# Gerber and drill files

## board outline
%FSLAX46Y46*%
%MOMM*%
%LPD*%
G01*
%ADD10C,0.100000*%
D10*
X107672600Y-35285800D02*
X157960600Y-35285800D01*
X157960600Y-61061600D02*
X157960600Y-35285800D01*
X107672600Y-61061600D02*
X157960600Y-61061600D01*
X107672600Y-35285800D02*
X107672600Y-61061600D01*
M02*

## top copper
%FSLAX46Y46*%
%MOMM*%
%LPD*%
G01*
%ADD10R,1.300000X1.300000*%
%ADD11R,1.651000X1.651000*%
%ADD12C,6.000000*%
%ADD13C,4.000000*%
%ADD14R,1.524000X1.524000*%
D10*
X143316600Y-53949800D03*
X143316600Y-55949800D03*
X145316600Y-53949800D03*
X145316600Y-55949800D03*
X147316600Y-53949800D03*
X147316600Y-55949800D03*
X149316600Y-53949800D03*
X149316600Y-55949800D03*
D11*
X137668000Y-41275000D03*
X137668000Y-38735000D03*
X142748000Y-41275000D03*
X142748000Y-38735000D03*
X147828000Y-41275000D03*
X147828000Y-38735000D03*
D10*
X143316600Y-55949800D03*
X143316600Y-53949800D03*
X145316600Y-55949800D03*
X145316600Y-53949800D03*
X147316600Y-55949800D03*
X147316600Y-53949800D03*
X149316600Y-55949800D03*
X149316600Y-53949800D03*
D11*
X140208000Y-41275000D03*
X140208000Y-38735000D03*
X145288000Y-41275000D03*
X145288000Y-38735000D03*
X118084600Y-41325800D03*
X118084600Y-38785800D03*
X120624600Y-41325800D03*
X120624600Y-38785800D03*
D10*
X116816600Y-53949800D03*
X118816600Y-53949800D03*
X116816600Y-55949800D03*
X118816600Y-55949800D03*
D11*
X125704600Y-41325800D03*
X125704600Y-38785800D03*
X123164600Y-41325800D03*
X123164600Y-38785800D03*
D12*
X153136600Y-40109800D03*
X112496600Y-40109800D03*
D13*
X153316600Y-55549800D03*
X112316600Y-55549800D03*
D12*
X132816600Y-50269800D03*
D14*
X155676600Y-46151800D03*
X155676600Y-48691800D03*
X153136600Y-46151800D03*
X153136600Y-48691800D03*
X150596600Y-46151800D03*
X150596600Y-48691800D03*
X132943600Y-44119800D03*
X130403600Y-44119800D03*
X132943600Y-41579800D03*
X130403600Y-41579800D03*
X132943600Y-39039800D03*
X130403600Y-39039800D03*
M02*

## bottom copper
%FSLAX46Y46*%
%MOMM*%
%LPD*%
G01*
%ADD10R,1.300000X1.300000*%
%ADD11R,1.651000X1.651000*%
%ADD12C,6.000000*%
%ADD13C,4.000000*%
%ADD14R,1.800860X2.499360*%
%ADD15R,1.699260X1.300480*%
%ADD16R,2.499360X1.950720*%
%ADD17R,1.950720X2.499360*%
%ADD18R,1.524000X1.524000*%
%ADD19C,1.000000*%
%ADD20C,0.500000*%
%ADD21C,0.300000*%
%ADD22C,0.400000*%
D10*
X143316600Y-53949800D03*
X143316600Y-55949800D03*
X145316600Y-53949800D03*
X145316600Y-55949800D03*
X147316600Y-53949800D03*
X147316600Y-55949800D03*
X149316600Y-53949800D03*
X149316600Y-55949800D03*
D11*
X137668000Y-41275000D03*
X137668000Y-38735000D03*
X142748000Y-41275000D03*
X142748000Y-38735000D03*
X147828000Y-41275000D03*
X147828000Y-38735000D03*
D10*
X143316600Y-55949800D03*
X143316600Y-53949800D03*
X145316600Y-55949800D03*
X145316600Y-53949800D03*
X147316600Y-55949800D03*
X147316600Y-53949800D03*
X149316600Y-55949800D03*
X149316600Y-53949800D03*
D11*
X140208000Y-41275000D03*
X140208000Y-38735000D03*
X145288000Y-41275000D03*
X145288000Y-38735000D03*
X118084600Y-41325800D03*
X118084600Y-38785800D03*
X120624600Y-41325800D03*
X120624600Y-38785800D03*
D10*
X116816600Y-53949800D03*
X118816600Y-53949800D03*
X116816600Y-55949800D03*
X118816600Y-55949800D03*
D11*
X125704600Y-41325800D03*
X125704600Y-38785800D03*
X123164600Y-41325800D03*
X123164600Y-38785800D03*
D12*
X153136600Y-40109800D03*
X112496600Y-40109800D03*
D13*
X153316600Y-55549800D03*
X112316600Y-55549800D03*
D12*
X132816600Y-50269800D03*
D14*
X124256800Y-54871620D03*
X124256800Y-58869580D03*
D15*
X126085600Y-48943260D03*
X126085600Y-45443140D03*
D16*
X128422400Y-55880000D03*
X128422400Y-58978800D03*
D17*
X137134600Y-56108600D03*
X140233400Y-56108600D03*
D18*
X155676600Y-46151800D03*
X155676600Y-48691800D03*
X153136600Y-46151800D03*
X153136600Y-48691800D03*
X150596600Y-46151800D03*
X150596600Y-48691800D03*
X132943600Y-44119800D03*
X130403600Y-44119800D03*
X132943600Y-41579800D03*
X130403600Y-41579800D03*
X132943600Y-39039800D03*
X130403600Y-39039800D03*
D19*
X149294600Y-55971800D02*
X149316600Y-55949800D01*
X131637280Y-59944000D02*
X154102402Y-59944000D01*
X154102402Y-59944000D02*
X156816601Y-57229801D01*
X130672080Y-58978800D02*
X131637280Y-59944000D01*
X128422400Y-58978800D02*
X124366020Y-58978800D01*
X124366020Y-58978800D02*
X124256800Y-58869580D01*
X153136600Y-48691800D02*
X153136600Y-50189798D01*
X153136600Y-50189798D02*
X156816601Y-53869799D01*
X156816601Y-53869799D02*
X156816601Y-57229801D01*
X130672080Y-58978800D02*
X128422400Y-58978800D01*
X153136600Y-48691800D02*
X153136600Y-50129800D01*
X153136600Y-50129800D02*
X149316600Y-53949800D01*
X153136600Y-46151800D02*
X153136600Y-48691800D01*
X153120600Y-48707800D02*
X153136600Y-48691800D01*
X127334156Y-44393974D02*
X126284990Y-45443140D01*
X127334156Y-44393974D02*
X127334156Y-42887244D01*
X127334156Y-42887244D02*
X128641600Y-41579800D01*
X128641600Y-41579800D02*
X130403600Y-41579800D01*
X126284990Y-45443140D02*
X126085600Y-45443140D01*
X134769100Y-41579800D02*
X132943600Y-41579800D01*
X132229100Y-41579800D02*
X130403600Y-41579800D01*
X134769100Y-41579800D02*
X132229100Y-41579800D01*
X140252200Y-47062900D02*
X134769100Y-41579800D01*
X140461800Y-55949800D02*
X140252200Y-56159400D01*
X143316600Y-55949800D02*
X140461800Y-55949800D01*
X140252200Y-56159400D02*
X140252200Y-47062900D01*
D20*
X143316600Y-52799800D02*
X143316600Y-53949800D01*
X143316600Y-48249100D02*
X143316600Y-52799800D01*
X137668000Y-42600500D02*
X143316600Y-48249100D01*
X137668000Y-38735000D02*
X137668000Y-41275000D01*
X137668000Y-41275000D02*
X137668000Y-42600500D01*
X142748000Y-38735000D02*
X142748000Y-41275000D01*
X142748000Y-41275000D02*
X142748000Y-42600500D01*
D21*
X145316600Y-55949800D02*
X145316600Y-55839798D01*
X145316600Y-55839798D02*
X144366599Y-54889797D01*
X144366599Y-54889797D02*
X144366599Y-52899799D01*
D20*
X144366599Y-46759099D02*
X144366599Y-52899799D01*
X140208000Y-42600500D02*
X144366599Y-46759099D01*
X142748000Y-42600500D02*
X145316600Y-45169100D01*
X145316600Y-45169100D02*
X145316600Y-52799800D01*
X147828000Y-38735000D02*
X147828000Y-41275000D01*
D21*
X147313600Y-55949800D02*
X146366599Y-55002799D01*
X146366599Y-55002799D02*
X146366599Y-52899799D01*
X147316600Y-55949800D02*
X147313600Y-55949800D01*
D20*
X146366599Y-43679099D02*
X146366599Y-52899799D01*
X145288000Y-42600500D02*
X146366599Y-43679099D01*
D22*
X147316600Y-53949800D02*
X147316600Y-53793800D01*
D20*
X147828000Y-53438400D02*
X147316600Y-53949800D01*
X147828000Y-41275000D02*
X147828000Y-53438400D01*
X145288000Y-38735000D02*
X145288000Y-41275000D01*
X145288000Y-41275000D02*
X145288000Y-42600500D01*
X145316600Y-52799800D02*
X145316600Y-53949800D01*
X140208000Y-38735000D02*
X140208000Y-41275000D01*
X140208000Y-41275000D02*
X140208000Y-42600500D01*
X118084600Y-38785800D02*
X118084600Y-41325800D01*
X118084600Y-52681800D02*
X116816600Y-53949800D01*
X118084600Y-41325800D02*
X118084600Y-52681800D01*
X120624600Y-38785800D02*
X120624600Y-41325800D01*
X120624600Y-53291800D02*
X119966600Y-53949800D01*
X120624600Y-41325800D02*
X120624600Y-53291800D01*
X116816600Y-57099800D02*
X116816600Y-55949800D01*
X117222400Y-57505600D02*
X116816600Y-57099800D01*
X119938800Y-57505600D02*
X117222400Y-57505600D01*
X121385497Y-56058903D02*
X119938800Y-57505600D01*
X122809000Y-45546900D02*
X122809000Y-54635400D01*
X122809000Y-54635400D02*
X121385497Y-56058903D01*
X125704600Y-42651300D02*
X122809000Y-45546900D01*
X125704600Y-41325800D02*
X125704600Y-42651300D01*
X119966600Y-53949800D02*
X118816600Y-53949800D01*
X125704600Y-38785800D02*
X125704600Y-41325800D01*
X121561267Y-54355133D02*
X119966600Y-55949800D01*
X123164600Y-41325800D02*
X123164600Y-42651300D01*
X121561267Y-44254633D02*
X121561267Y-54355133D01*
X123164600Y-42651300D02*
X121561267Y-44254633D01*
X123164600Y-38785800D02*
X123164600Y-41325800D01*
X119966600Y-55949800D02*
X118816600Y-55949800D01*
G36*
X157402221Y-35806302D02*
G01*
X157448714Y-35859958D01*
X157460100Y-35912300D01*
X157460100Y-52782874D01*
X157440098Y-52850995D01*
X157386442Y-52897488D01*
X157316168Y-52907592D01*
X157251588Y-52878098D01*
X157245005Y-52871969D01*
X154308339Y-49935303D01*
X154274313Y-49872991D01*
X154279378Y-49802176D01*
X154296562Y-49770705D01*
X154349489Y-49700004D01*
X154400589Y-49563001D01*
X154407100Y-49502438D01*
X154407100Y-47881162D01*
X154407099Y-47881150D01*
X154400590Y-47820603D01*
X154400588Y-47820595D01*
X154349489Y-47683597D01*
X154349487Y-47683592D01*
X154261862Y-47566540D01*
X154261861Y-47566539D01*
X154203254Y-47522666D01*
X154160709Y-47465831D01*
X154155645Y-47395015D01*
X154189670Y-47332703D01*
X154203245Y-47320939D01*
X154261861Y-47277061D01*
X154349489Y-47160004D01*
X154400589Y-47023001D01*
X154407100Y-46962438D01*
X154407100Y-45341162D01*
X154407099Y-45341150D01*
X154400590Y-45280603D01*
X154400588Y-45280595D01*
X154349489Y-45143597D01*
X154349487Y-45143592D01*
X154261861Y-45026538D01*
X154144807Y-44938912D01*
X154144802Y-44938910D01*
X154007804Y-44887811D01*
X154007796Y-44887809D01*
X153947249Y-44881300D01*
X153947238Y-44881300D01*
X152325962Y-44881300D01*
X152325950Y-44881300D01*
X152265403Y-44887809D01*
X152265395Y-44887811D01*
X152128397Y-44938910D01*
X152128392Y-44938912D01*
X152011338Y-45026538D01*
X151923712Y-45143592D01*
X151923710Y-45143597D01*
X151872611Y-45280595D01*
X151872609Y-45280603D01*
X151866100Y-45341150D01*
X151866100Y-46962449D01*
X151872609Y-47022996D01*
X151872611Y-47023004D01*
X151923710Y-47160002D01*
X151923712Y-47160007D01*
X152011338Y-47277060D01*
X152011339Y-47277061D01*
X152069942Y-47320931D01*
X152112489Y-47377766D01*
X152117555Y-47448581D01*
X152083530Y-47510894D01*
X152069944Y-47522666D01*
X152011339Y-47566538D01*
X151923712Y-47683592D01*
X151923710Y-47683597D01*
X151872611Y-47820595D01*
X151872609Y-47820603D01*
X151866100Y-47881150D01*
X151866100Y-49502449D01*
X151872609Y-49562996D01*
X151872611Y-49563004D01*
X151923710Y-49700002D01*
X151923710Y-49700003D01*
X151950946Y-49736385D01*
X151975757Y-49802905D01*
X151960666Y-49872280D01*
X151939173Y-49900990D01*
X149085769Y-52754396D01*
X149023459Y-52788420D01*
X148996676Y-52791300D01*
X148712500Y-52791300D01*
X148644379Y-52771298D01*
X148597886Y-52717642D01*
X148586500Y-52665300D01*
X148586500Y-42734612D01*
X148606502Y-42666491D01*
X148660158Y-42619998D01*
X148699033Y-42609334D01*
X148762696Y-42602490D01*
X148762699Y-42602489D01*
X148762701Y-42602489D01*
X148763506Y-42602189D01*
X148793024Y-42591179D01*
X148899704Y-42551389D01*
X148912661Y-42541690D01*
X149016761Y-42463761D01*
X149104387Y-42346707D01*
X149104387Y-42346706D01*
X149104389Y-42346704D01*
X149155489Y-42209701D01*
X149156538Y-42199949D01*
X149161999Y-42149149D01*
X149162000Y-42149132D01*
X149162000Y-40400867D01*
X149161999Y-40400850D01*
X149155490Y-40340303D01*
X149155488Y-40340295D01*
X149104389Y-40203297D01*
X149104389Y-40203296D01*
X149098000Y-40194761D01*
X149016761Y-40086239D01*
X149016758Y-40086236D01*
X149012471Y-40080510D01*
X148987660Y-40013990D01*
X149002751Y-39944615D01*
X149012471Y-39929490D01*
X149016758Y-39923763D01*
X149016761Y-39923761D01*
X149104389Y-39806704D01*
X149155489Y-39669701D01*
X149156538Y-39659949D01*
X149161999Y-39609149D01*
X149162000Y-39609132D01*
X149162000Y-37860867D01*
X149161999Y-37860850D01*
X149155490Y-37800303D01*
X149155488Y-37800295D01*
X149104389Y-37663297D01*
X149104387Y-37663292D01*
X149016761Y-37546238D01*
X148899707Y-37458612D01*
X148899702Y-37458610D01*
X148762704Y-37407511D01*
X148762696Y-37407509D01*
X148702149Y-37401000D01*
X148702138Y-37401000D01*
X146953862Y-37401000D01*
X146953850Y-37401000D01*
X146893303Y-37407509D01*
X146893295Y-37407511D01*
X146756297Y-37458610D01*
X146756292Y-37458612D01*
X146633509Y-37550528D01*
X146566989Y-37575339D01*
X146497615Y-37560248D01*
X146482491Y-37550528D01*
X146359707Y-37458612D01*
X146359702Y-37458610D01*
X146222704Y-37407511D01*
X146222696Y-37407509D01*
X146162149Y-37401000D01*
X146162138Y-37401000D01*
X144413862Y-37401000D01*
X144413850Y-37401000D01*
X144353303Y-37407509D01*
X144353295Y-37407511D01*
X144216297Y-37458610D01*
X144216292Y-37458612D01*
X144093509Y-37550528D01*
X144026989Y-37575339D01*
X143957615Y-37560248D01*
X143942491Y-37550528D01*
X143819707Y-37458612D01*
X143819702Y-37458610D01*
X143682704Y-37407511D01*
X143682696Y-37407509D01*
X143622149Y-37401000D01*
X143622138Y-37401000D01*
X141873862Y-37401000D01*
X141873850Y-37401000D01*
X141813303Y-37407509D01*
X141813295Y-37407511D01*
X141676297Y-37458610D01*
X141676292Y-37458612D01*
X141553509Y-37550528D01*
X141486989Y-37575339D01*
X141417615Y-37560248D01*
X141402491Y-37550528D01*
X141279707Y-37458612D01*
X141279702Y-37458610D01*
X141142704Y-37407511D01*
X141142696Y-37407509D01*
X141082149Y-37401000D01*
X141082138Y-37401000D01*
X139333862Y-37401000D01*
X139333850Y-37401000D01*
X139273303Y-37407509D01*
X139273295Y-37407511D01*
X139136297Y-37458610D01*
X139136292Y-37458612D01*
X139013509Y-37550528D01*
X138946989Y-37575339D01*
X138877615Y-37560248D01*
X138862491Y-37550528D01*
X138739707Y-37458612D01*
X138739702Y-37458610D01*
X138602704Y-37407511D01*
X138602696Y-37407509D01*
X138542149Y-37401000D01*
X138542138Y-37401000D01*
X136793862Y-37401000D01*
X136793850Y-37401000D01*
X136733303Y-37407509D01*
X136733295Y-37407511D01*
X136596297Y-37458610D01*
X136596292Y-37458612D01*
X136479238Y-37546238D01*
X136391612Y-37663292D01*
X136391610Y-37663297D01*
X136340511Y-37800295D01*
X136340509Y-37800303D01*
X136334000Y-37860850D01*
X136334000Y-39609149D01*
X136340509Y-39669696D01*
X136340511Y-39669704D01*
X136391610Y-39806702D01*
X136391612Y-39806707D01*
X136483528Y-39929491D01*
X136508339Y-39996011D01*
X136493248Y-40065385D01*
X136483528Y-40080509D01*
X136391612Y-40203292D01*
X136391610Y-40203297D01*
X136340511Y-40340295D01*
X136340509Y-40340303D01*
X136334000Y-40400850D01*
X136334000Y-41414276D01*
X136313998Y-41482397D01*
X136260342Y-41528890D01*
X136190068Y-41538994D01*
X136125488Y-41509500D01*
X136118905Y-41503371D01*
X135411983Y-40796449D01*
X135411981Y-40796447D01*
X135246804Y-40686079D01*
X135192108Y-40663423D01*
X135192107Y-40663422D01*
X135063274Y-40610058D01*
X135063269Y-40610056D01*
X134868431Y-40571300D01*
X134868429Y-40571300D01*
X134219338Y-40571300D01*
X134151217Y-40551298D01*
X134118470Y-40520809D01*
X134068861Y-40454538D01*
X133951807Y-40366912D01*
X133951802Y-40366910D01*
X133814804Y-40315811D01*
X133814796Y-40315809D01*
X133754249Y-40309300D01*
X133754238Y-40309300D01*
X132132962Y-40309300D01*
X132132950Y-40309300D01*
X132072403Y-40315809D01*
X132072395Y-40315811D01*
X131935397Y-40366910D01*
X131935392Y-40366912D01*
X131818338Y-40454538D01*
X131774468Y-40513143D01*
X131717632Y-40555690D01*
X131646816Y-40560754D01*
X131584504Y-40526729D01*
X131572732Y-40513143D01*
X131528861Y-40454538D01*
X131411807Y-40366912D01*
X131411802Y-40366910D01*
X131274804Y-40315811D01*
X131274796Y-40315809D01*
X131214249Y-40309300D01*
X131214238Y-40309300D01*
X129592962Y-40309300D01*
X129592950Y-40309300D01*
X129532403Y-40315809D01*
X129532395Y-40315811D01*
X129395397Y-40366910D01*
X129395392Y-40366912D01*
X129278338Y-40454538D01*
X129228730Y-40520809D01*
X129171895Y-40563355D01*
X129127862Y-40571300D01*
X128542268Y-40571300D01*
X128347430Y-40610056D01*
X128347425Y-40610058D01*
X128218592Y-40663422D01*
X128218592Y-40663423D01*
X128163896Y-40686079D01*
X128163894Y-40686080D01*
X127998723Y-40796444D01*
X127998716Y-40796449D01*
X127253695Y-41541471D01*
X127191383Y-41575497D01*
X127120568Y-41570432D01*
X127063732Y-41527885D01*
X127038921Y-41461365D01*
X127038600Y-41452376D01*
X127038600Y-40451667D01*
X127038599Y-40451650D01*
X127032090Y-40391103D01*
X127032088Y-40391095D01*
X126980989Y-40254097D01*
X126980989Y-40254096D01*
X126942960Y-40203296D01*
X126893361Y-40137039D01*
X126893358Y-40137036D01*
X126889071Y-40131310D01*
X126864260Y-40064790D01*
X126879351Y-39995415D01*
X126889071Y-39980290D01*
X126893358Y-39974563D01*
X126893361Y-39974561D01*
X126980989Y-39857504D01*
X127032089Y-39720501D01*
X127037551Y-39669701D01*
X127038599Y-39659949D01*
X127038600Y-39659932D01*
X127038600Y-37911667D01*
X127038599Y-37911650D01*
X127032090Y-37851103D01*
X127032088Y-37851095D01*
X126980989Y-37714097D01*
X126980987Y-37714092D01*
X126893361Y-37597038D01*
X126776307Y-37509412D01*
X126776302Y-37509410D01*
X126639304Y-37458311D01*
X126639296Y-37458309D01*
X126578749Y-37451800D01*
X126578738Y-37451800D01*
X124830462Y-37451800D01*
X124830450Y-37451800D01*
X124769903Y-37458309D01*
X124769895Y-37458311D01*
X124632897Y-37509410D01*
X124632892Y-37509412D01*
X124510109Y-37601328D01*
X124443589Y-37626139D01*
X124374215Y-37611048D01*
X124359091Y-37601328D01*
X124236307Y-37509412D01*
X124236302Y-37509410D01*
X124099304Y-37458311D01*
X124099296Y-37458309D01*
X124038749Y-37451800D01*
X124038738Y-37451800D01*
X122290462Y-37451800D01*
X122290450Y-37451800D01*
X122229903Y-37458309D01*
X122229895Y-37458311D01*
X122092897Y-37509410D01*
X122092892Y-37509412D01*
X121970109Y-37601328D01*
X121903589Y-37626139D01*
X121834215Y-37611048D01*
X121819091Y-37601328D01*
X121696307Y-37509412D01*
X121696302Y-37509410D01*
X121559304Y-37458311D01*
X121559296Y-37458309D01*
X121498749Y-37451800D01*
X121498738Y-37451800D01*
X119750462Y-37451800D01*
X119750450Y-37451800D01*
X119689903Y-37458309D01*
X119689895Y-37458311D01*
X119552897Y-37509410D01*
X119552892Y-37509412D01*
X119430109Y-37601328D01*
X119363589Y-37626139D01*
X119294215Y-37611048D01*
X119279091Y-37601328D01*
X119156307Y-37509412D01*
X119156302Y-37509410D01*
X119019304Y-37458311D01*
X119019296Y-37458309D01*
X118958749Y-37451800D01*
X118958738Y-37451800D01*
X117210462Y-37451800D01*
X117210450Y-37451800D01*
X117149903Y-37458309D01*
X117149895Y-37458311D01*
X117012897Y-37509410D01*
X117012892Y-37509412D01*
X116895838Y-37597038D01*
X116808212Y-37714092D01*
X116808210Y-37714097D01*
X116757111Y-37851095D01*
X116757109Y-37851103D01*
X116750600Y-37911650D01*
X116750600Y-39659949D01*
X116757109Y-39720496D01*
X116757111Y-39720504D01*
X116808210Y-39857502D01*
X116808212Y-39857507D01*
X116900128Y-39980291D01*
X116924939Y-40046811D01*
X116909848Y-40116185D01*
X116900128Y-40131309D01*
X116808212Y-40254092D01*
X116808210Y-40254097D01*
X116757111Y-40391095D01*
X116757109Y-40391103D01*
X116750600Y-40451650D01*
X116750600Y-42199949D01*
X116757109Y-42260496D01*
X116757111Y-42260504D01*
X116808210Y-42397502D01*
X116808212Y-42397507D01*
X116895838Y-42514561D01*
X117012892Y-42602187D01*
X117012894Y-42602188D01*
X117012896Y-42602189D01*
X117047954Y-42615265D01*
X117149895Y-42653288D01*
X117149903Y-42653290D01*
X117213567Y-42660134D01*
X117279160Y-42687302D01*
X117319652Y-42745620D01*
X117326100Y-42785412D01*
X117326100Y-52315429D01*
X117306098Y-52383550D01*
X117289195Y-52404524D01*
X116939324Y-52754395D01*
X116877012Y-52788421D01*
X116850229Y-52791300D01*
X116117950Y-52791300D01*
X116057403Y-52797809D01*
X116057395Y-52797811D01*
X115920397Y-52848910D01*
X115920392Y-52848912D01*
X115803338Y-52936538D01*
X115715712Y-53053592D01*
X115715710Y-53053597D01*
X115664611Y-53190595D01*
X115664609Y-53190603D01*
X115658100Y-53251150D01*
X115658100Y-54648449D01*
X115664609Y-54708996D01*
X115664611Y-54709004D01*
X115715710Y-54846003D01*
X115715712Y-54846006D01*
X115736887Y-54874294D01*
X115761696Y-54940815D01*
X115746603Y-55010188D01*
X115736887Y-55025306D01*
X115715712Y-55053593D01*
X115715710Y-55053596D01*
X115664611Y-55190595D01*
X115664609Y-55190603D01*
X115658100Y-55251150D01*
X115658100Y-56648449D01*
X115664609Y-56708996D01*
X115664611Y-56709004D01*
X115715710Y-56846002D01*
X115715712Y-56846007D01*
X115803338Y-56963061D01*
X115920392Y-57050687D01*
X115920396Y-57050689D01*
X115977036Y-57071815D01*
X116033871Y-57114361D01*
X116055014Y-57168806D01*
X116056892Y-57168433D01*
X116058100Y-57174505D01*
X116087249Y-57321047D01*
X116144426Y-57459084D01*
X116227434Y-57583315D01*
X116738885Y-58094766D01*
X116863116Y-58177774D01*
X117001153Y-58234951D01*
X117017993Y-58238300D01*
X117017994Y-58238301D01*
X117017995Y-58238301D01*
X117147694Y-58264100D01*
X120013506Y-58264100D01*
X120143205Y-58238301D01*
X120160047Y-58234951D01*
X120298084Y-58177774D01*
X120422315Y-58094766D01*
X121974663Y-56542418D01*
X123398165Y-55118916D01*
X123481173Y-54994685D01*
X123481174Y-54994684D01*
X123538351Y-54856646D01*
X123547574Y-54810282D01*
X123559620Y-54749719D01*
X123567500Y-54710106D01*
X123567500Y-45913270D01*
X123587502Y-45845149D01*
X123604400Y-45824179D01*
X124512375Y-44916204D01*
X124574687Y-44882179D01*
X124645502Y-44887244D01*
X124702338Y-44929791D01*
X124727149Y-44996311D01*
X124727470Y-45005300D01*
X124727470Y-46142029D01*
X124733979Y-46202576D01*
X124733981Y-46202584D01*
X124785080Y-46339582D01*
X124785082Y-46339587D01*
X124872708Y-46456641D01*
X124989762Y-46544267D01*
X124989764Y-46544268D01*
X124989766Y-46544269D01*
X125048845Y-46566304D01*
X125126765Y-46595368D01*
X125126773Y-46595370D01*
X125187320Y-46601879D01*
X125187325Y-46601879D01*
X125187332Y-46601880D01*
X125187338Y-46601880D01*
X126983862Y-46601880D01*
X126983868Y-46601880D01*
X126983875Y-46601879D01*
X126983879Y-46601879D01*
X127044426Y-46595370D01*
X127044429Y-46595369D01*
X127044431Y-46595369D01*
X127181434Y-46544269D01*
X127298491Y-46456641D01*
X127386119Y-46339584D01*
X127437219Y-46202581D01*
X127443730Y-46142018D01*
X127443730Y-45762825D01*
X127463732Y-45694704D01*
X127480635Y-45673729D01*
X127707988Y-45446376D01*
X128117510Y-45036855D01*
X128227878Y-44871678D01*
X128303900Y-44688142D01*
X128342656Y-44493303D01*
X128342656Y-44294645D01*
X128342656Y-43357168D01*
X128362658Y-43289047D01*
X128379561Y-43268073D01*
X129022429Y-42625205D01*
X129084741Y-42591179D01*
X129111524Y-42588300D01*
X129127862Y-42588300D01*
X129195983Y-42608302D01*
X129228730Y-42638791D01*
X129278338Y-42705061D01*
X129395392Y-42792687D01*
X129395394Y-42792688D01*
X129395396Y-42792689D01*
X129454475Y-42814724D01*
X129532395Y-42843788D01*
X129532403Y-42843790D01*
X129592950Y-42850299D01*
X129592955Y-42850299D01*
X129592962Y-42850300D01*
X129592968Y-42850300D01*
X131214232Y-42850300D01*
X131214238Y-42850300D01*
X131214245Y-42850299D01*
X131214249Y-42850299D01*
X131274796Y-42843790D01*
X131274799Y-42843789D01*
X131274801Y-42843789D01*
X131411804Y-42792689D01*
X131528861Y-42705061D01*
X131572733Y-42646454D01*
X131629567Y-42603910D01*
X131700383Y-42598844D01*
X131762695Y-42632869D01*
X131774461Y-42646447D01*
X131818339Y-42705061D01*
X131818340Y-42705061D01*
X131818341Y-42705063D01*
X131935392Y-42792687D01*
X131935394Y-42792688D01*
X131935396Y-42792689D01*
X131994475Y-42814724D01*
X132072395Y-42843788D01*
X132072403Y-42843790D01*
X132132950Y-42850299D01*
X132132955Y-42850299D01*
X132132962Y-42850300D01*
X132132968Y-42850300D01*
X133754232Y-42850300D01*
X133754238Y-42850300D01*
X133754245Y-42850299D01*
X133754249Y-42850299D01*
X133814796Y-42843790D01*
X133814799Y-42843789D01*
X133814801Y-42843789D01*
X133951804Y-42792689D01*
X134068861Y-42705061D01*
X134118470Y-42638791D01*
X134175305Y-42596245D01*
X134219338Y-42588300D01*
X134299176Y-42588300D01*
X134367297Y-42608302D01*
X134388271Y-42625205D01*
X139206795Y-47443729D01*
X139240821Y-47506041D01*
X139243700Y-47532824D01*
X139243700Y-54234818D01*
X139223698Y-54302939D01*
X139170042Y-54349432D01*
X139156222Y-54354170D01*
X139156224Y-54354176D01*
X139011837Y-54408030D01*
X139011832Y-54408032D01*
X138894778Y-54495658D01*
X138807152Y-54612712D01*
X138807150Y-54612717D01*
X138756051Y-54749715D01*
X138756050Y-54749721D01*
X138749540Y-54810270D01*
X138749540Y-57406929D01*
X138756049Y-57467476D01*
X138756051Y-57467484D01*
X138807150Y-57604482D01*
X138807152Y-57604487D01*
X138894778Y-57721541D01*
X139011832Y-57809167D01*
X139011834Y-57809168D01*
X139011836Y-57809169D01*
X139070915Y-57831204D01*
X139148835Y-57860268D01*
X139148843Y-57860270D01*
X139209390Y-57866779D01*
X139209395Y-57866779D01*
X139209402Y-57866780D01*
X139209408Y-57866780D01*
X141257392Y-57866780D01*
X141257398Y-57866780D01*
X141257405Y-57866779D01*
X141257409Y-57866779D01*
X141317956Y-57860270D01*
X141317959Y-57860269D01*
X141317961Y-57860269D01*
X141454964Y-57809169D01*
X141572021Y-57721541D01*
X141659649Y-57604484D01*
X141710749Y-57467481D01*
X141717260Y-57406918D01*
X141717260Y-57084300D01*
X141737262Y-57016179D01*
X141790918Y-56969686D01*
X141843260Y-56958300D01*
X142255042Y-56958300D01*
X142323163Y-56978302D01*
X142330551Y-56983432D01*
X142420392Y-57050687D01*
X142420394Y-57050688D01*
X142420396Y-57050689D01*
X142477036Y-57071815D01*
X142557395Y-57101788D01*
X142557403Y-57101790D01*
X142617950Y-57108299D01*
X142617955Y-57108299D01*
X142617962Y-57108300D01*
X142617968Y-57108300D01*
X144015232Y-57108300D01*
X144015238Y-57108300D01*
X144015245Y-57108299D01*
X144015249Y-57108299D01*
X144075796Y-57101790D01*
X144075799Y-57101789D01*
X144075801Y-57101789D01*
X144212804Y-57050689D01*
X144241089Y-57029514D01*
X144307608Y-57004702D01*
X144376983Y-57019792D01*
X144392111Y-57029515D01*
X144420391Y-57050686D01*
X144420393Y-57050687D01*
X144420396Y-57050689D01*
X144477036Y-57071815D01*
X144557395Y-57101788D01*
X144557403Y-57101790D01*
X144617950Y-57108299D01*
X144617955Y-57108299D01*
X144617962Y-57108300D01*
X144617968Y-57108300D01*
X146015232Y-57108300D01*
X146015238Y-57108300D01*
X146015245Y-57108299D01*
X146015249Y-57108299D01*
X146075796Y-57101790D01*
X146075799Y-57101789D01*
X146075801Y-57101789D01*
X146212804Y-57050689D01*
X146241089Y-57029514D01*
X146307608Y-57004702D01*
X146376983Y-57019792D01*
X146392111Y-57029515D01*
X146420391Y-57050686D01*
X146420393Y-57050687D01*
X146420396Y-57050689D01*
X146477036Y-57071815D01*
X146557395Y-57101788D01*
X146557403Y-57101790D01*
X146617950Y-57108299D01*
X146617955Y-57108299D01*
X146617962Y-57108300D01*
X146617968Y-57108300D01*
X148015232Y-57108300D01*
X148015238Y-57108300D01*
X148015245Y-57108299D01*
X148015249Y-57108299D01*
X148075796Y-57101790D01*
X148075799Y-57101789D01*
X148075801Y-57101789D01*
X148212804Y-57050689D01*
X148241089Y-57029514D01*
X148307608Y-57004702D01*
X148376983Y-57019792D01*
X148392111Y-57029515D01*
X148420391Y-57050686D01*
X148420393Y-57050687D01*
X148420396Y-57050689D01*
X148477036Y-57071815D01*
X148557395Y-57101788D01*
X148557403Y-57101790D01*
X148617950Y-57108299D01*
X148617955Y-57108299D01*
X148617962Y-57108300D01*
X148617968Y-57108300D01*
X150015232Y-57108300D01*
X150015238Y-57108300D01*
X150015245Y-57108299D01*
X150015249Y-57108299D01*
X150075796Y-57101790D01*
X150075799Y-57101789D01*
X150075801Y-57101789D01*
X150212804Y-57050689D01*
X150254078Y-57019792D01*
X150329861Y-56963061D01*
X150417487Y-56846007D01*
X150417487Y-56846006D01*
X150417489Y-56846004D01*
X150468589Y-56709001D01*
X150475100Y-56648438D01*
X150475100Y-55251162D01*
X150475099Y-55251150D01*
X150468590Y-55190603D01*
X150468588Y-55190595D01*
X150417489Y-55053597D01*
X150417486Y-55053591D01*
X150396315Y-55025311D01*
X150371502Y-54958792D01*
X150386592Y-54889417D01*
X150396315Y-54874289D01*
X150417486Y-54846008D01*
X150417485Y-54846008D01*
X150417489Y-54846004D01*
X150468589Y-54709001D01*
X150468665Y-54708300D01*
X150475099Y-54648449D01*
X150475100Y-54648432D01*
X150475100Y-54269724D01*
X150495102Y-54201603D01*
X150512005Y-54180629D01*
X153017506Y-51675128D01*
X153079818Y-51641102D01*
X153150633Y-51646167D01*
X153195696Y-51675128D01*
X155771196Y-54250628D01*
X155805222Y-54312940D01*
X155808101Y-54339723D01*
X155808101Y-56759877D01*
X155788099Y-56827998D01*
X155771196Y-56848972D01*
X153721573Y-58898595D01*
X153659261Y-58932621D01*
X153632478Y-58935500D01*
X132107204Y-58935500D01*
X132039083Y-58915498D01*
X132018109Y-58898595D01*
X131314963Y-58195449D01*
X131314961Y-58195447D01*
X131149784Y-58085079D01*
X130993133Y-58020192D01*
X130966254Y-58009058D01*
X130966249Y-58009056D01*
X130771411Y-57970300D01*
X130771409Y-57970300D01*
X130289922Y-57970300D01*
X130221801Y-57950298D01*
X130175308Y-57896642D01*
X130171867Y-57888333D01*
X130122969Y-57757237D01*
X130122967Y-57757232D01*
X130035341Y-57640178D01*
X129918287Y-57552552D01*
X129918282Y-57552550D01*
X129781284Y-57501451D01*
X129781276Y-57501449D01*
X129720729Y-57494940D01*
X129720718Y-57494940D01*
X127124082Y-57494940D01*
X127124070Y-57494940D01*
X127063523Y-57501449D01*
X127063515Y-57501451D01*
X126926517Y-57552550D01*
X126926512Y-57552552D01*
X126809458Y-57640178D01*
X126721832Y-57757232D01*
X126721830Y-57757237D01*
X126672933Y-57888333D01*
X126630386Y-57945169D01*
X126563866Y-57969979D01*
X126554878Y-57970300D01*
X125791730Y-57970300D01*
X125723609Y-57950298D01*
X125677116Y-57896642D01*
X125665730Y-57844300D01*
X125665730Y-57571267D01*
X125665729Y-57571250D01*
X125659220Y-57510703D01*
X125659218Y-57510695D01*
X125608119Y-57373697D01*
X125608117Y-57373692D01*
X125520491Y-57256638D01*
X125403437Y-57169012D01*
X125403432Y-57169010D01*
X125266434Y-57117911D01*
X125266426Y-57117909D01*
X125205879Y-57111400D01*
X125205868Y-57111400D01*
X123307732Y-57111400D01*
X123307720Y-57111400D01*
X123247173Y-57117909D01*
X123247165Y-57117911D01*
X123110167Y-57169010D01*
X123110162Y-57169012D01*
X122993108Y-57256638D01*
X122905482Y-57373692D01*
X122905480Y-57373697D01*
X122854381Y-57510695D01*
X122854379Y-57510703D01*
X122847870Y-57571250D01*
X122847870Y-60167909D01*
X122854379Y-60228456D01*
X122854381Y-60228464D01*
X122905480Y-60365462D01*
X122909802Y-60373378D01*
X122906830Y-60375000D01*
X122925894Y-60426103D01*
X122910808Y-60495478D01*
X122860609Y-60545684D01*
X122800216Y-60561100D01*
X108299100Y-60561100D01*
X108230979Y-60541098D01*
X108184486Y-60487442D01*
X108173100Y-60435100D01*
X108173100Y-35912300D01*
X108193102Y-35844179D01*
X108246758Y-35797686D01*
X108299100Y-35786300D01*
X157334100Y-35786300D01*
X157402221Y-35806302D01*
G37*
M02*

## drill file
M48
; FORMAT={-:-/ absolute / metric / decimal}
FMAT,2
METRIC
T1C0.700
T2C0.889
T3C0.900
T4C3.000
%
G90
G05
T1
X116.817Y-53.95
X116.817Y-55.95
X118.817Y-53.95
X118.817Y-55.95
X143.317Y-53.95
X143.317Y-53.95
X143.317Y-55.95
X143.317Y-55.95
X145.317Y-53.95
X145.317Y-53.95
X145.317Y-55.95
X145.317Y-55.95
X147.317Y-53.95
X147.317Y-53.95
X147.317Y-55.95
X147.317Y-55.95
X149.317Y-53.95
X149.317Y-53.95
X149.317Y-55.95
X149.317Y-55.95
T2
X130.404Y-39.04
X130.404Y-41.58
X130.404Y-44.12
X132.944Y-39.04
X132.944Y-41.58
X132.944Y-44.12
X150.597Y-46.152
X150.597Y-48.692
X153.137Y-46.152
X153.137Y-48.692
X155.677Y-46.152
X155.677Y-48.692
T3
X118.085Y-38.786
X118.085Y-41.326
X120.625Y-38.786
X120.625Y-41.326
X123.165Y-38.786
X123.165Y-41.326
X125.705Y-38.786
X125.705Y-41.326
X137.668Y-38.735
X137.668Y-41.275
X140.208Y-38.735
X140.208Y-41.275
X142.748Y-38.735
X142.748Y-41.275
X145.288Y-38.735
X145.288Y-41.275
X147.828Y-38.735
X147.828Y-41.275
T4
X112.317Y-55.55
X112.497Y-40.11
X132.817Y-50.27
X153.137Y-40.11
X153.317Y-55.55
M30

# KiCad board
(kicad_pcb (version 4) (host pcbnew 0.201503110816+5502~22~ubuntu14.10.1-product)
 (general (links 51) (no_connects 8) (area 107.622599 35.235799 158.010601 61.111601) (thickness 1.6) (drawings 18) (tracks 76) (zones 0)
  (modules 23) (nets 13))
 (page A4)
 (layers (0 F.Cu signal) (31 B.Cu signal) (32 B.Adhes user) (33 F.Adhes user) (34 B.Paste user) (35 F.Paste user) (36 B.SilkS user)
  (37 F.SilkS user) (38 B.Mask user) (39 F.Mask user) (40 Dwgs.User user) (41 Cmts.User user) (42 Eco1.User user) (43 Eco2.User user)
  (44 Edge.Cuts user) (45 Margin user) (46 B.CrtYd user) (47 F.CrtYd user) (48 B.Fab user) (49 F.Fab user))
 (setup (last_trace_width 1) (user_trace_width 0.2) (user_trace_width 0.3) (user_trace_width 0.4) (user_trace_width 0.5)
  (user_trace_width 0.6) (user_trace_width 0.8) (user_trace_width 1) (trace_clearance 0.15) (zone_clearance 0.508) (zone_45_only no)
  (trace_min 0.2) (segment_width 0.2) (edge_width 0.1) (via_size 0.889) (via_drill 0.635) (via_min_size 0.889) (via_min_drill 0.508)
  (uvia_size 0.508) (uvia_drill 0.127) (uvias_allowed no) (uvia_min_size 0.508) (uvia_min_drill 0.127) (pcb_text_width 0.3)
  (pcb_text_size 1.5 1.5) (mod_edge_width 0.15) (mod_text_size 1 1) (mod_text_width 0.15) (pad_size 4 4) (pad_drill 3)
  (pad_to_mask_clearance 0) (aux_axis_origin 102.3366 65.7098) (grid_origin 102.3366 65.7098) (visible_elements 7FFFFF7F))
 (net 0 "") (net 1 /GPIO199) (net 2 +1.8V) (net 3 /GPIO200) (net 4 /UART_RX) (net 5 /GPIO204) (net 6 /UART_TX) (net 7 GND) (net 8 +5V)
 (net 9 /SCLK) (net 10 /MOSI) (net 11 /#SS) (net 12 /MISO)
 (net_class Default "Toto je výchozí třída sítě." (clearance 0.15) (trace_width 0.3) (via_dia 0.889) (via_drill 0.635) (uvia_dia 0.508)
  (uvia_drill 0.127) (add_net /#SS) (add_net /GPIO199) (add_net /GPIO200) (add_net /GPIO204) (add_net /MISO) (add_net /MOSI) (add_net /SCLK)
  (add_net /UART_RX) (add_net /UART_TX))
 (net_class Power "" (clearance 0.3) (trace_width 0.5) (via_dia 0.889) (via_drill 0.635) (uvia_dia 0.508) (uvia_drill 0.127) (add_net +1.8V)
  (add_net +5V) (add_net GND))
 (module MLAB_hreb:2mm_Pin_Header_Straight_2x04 (layer B.Cu) (at 146.3166 54.9498 270)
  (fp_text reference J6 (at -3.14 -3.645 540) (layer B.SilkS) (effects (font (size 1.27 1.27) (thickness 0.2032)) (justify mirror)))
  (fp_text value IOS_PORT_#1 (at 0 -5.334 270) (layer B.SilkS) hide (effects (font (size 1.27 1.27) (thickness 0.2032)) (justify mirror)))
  (pad 1 thru_hole rect (at -1 3 270) (size 1.3 1.3) (drill 0.7) (layers *.Cu *.Mask B.SilkS) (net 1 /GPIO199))
  (pad 2 thru_hole rect (at 1 3 270) (size 1.3 1.3) (drill 0.7) (layers *.Cu *.Mask B.SilkS) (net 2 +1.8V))
  (pad 3 thru_hole rect (at -1 1 270) (size 1.3 1.3) (drill 0.7) (layers *.Cu *.Mask B.SilkS) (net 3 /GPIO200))
  (pad 4 thru_hole rect (at 1 1 270) (size 1.3 1.3) (drill 0.7) (layers *.Cu *.Mask B.SilkS) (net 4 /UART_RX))
  (pad 5 thru_hole rect (at -1 -1 270) (size 1.3 1.3) (drill 0.7) (layers *.Cu *.Mask B.SilkS) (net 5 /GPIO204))
  (pad 6 thru_hole rect (at 1 -1 270) (size 1.3 1.3) (drill 0.7) (layers *.Cu *.Mask B.SilkS) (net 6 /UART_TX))
  (pad 7 thru_hole rect (at -1 -3 270) (size 1.3 1.3) (drill 0.7) (layers *.Cu *.Mask B.SilkS) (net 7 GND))
  (pad 8 thru_hole rect (at 1 -3 270) (size 1.3 1.3) (drill 0.7) (layers *.Cu *.Mask B.SilkS) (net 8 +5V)))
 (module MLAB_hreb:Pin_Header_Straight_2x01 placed (layer F.Cu) (at 137.668 40.005)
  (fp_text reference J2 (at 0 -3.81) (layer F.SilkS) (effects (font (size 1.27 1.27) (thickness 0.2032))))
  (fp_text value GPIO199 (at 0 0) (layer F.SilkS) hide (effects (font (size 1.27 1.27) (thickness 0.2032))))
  (pad 2 thru_hole rect (at 0 1.27) (size 1.651 1.651) (drill 0.9) (layers *.Cu *.Mask F.SilkS) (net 1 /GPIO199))
  (pad 1 thru_hole rect (at 0 -1.27) (size 1.651 1.651) (drill 0.9) (layers *.Cu *.Mask F.SilkS) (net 1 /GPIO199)))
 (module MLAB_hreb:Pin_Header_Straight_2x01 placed (layer F.Cu) (at 142.748 40.005)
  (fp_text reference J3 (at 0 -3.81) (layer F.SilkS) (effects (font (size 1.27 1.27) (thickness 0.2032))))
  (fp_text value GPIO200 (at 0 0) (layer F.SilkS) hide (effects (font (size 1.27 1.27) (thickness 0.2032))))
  (pad 2 thru_hole rect (at 0 1.27) (size 1.651 1.651) (drill 0.9) (layers *.Cu *.Mask F.SilkS) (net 3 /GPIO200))
  (pad 1 thru_hole rect (at 0 -1.27) (size 1.651 1.651) (drill 0.9) (layers *.Cu *.Mask F.SilkS) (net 3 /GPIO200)))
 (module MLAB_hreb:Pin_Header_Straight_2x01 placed (layer F.Cu) (at 147.828 40.005)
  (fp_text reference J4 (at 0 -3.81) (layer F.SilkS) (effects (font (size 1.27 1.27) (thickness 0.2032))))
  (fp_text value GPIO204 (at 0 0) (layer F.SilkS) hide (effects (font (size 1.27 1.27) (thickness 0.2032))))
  (pad 2 thru_hole rect (at 0 1.27) (size 1.651 1.651) (drill 0.9) (layers *.Cu *.Mask F.SilkS) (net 5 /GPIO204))
  (pad 1 thru_hole rect (at 0 -1.27) (size 1.651 1.651) (drill 0.9) (layers *.Cu *.Mask F.SilkS) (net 5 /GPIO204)))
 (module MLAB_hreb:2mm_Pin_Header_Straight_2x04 (layer F.Cu) (at 146.3166 54.9498 90)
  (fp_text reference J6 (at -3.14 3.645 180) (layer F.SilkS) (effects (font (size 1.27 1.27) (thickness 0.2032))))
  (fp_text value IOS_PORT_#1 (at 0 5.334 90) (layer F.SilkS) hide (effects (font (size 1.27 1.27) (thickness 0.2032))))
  (pad 1 thru_hole rect (at -1 -3 90) (size 1.3 1.3) (drill 0.7) (layers *.Cu *.Mask F.SilkS) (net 1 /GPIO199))
  (pad 2 thru_hole rect (at 1 -3 90) (size 1.3 1.3) (drill 0.7) (layers *.Cu *.Mask F.SilkS) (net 2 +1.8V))
  (pad 3 thru_hole rect (at -1 -1 90) (size 1.3 1.3) (drill 0.7) (layers *.Cu *.Mask F.SilkS) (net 3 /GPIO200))
  (pad 4 thru_hole rect (at 1 -1 90) (size 1.3 1.3) (drill 0.7) (layers *.Cu *.Mask F.SilkS) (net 4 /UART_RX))
  (pad 5 thru_hole rect (at -1 1 90) (size 1.3 1.3) (drill 0.7) (layers *.Cu *.Mask F.SilkS) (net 5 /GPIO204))
  (pad 6 thru_hole rect (at 1 1 90) (size 1.3 1.3) (drill 0.7) (layers *.Cu *.Mask F.SilkS) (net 6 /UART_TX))
  (pad 7 thru_hole rect (at -1 3 90) (size 1.3 1.3) (drill 0.7) (layers *.Cu *.Mask F.SilkS) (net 7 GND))
  (pad 8 thru_hole rect (at 1 3 90) (size 1.3 1.3) (drill 0.7) (layers *.Cu *.Mask F.SilkS) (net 8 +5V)))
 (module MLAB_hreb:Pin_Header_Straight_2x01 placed (layer F.Cu) (at 140.208 40.005)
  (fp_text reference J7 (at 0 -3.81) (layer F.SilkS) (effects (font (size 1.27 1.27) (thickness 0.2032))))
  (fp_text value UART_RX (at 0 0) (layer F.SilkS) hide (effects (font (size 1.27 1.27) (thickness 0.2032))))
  (pad 2 thru_hole rect (at 0 1.27) (size 1.651 1.651) (drill 0.9) (layers *.Cu *.Mask F.SilkS) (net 4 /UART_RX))
  (pad 1 thru_hole rect (at 0 -1.27) (size 1.651 1.651) (drill 0.9) (layers *.Cu *.Mask F.SilkS) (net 4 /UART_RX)))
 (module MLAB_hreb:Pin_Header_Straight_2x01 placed (layer F.Cu) (at 145.288 40.005)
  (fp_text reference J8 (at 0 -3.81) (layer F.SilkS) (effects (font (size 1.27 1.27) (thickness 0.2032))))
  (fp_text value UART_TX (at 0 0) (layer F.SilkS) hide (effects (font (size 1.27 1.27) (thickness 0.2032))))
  (pad 2 thru_hole rect (at 0 1.27) (size 1.651 1.651) (drill 0.9) (layers *.Cu *.Mask F.SilkS) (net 6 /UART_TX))
  (pad 1 thru_hole rect (at 0 -1.27) (size 1.651 1.651) (drill 0.9) (layers *.Cu *.Mask F.SilkS) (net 6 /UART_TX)))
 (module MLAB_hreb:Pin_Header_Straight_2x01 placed (layer F.Cu) (at 118.0846 40.0558)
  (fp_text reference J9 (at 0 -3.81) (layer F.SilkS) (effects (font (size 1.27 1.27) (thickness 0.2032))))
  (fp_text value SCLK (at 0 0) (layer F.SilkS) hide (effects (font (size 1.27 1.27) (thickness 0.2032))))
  (pad 2 thru_hole rect (at 0 1.27) (size 1.651 1.651) (drill 0.9) (layers *.Cu *.Mask F.SilkS) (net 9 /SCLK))
  (pad 1 thru_hole rect (at 0 -1.27) (size 1.651 1.651) (drill 0.9) (layers *.Cu *.Mask F.SilkS) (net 9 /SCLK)))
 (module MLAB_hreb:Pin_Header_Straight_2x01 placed (layer F.Cu) (at 120.6246 40.0558)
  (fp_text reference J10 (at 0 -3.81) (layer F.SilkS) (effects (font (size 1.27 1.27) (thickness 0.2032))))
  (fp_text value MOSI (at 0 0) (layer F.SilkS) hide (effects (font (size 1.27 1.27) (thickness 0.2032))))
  (pad 2 thru_hole rect (at 0 1.27) (size 1.651 1.651) (drill 0.9) (layers *.Cu *.Mask F.SilkS) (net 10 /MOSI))
  (pad 1 thru_hole rect (at 0 -1.27) (size 1.651 1.651) (drill 0.9) (layers *.Cu *.Mask F.SilkS) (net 10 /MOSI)))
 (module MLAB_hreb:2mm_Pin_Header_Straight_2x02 (layer F.Cu) (at 117.8166 54.9498)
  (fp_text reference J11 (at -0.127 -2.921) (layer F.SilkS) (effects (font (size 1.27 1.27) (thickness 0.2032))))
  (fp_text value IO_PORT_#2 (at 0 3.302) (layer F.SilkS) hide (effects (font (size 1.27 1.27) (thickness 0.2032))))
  (pad 1 thru_hole rect (at -1 -1) (size 1.3 1.3) (drill 0.7) (layers *.Cu *.Mask F.SilkS) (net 9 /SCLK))
  (pad 2 thru_hole rect (at 1 -1) (size 1.3 1.3) (drill 0.7) (layers *.Cu *.Mask F.SilkS) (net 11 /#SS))
  (pad 3 thru_hole rect (at -1 1) (size 1.3 1.3) (drill 0.7) (layers *.Cu *.Mask F.SilkS) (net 10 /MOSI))
  (pad 4 thru_hole rect (at 1 1) (size 1.3 1.3) (drill 0.7) (layers *.Cu *.Mask F.SilkS) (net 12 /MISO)))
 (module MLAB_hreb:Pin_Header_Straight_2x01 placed (layer F.Cu) (at 125.7046 40.0558)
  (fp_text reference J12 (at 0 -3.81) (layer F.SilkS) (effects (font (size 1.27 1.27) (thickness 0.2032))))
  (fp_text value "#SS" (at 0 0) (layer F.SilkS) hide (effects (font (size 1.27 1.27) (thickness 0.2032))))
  (pad 2 thru_hole rect (at 0 1.27) (size 1.651 1.651) (drill 0.9) (layers *.Cu *.Mask F.SilkS) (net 11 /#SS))
  (pad 1 thru_hole rect (at 0 -1.27) (size 1.651 1.651) (drill 0.9) (layers *.Cu *.Mask F.SilkS) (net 11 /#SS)))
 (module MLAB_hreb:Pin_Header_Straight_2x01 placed (layer F.Cu) (at 123.1646 40.0558)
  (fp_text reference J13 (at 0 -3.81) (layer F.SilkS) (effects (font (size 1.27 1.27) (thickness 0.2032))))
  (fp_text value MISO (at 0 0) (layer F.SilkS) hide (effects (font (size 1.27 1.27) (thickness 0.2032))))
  (pad 2 thru_hole rect (at 0 1.27) (size 1.651 1.651) (drill 0.9) (layers *.Cu *.Mask F.SilkS) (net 12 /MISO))
  (pad 1 thru_hole rect (at 0 -1.27) (size 1.651 1.651) (drill 0.9) (layers *.Cu *.Mask F.SilkS) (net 12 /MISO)))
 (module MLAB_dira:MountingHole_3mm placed (layer F.Cu) (at 153.1366 40.1098)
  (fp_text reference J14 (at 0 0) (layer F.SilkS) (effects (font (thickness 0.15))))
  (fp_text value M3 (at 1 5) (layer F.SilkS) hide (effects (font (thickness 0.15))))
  (pad 1 thru_hole circle (at 0 0) (size 6 6) (drill 3) (layers *.Cu *.Adhes *.Mask) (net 7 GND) (clearance 1) (zone_connect 2)))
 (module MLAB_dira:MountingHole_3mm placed (layer F.Cu) (at 112.4966 40.1098)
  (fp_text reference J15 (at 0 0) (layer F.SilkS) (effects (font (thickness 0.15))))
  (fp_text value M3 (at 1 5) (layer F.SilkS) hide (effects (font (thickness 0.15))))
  (pad 1 thru_hole circle (at 0 0) (size 6 6) (drill 3) (layers *.Cu *.Adhes *.Mask) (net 7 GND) (clearance 1) (zone_connect 2)))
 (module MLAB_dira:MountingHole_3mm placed (layer F.Cu) (at 153.3166 55.5498)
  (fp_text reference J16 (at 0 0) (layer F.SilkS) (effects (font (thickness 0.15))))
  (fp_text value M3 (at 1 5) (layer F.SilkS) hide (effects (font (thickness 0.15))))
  (pad 1 thru_hole circle (at 0 0) (size 4 4) (drill 3) (layers *.Cu *.Adhes *.Mask) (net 7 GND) (clearance 1) (zone_connect 2)))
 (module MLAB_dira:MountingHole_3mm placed (layer F.Cu) (at 112.3166 55.5498)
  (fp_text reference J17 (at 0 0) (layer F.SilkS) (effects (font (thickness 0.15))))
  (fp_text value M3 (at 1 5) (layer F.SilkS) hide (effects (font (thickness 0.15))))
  (pad 1 thru_hole circle (at 0 0) (size 4 4) (drill 3) (layers *.Cu *.Adhes *.Mask) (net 7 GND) (clearance 1) (zone_connect 2)))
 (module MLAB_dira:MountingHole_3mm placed (layer F.Cu) (at 132.8166 50.2698)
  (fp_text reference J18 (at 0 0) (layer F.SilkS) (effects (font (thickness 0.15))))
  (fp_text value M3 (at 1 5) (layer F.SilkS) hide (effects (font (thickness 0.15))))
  (pad 1 thru_hole circle (at 0 0) (size 6 6) (drill 3) (layers *.Cu *.Adhes *.Mask) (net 7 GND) (clearance 1) (zone_connect 2)))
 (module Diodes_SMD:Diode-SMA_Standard (layer B.Cu) (at 124.2568 56.8706 270)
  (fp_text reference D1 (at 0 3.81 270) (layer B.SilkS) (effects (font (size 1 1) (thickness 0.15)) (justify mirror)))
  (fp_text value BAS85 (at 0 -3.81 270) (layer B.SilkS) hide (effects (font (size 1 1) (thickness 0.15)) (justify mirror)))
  (pad 1 smd rect (at -1.99898 0 270) (size 2.49936 1.80086) (layers B.Cu B.Paste B.Mask) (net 7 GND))
  (pad 2 smd rect (at 1.99898 0 270) (size 2.49936 1.80086) (layers B.Cu B.Paste B.Mask) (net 8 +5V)))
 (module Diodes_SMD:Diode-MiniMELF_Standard (layer B.Cu) (at 126.0856 47.1932 90)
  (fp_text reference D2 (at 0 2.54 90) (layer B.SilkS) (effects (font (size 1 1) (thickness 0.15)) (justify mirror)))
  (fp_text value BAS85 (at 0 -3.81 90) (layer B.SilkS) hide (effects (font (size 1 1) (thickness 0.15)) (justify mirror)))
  (pad 1 smd rect (at -1.75006 0 90) (size 1.30048 1.69926) (layers B.Cu B.Paste B.Mask) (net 7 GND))
  (pad 2 smd rect (at 1.75006 0 90) (size 1.30048 1.69926) (layers B.Cu B.Paste B.Mask) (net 2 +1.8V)))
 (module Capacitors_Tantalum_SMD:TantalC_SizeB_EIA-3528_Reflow (layer B.Cu) (at 128.4224 57.4294 90)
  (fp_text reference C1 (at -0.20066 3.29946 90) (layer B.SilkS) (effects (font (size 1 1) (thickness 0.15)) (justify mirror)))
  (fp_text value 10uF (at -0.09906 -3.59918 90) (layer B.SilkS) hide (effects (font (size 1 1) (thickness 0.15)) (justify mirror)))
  (pad 2 smd rect (at 1.5494 0 90) (size 1.95072 2.49936) (layers B.Cu B.Paste B.Mask) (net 7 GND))
  (pad 1 smd rect (at -1.5494 0 90) (size 1.95072 2.49936) (layers B.Cu B.Paste B.Mask) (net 8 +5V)))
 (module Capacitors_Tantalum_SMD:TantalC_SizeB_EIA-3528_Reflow (layer B.Cu) (at 138.684 56.1086 180)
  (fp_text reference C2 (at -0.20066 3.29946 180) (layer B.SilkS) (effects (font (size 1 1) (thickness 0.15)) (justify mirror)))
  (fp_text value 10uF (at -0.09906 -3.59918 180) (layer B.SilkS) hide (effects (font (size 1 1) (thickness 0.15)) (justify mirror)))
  (pad 2 smd rect (at 1.5494 0 180) (size 1.95072 2.49936) (layers B.Cu B.Paste B.Mask) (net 7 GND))
  (pad 1 smd rect (at -1.5494 0 180) (size 1.95072 2.49936) (layers B.Cu B.Paste B.Mask) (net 2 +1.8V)))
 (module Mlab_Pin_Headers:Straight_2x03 (layer F.Cu) (at 153.1366 47.4218 270)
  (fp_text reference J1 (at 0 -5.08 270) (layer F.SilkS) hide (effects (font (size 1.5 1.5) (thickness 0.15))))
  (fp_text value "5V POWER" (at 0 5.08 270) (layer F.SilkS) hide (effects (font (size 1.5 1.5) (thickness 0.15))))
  (pad 1 thru_hole rect (at -1.27 -2.54 270) (size 1.524 1.524) (drill 0.889) (layers *.Cu *.Mask F.SilkS) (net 7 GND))
  (pad 2 thru_hole rect (at 1.27 -2.54 270) (size 1.524 1.524) (drill 0.889) (layers *.Cu *.Mask F.SilkS) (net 7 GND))
  (pad 3 thru_hole rect (at -1.27 0 270) (size 1.524 1.524) (drill 0.889) (layers *.Cu *.Mask F.SilkS) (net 8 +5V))
  (pad 4 thru_hole rect (at 1.27 0 270) (size 1.524 1.524) (drill 0.889) (layers *.Cu *.Mask F.SilkS) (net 8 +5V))
  (pad 5 thru_hole rect (at -1.27 2.54 270) (size 1.524 1.524) (drill 0.889) (layers *.Cu *.Mask F.SilkS) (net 7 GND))
  (pad 6 thru_hole rect (at 1.27 2.54 270) (size 1.524 1.524) (drill 0.889) (layers *.Cu *.Mask F.SilkS) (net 7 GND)))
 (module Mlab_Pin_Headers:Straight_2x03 (layer F.Cu) (at 131.6736 41.5798 180)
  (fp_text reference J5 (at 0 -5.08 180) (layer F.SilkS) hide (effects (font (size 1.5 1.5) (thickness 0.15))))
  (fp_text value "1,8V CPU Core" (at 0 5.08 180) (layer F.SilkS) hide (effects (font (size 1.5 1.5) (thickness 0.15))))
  (pad 1 thru_hole rect (at -1.27 -2.54 180) (size 1.524 1.524) (drill 0.889) (layers *.Cu *.Mask F.SilkS) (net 7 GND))
  (pad 2 thru_hole rect (at 1.27 -2.54 180) (size 1.524 1.524) (drill 0.889) (layers *.Cu *.Mask F.SilkS) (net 7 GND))
  (pad 3 thru_hole rect (at -1.27 0 180) (size 1.524 1.524) (drill 0.889) (layers *.Cu *.Mask F.SilkS) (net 2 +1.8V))
  (pad 4 thru_hole rect (at 1.27 0 180) (size 1.524 1.524) (drill 0.889) (layers *.Cu *.Mask F.SilkS) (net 2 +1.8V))
  (pad 5 thru_hole rect (at -1.27 2.54 180) (size 1.524 1.524) (drill 0.889) (layers *.Cu *.Mask F.SilkS) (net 7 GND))
  (pad 6 thru_hole rect (at 1.27 2.54 180) (size 1.524 1.524) (drill 0.889) (layers *.Cu *.Mask F.SilkS) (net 7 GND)))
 (gr_line (start 107.6726 35.2858) (end 157.9606 35.2858) (angle 90) (layer Edge.Cuts) (width 0.1))
 (gr_line (start 157.9606 61.0616) (end 157.9606 35.2858) (angle 90) (layer Edge.Cuts) (width 0.1))
 (gr_line (start 107.6726 61.0616) (end 157.9606 61.0616) (angle 90) (layer Edge.Cuts) (width 0.1))
 (gr_line (start 107.6726 35.2858) (end 107.6726 61.0616) (angle 90) (layer Edge.Cuts) (width 0.1))
 (segment (start 149.2946 55.9718) (end 149.3166 55.9498) (width 1) (layer B.Cu) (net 7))
 (segment (start 131.63728 59.944) (end 154.102402 59.944) (width 1) (layer B.Cu) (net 8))
 (segment (start 154.102402 59.944) (end 156.816601 57.229801) (width 1) (layer B.Cu) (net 8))
 (segment (start 130.67208 58.9788) (end 131.63728 59.944) (width 1) (layer B.Cu) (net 8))
 (segment (start 128.4224 58.9788) (end 124.36602 58.9788) (width 1) (layer B.Cu) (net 8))
 (segment (start 124.36602 58.9788) (end 124.2568 58.86958) (width 1) (layer B.Cu) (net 8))
 (segment (start 153.1366 48.6918) (end 153.1366 50.189798) (width 1) (layer B.Cu) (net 8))
 (segment (start 153.1366 50.189798) (end 156.816601 53.869799) (width 1) (layer B.Cu) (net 8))
 (segment (start 156.816601 53.869799) (end 156.816601 57.229801) (width 1) (layer B.Cu) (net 8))
 (segment (start 130.67208 58.9788) (end 128.4224 58.9788) (width 1) (layer B.Cu) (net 8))
 (segment (start 153.1366 48.6918) (end 153.1366 50.1298) (width 1) (layer B.Cu) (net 8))
 (segment (start 153.1366 50.1298) (end 149.3166 53.9498) (width 1) (layer B.Cu) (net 8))
 (segment (start 153.1366 46.1518) (end 153.1366 48.6918) (width 1) (layer B.Cu) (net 8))
 (segment (start 153.1206 48.7078) (end 153.1366 48.6918) (width 1) (layer B.Cu) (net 8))
 (segment (start 127.334156 44.393974) (end 126.28499 45.44314) (width 1) (layer B.Cu) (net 2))
 (segment (start 127.334156 44.393974) (end 127.334156 42.887244) (width 1) (layer B.Cu) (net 2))
 (segment (start 127.334156 42.887244) (end 128.6416 41.5798) (width 1) (layer B.Cu) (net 2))
 (segment (start 128.6416 41.5798) (end 130.4036 41.5798) (width 1) (layer B.Cu) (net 2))
 (segment (start 126.28499 45.44314) (end 126.0856 45.44314) (width 1) (layer B.Cu) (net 2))
 (segment (start 134.7691 41.5798) (end 132.9436 41.5798) (width 1) (layer B.Cu) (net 2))
 (segment (start 132.2291 41.5798) (end 130.4036 41.5798) (width 1) (layer B.Cu) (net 2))
 (segment (start 134.7691 41.5798) (end 132.2291 41.5798) (width 1) (layer B.Cu) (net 2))
 (segment (start 140.2522 47.0629) (end 134.7691 41.5798) (width 1) (layer B.Cu) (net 2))
 (segment (start 140.4618 55.9498) (end 140.2522 56.1594) (width 1) (layer B.Cu) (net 2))
 (segment (start 143.3166 55.9498) (end 140.4618 55.9498) (width 1) (layer B.Cu) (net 2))
 (segment (start 140.2522 56.1594) (end 140.2522 47.0629) (width 1) (layer B.Cu) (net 2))
 (segment (start 143.3166 52.7998) (end 143.3166 53.9498) (width 0.5) (layer B.Cu) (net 2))
 (segment (start 143.3166 48.2491) (end 143.3166 52.7998) (width 0.5) (layer B.Cu) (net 2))
 (segment (start 137.668 42.6005) (end 143.3166 48.2491) (width 0.5) (layer B.Cu) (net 2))
 (segment (start 137.668 38.735) (end 137.668 41.275) (width 0.5) (layer B.Cu) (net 1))
 (segment (start 137.668 41.275) (end 137.668 42.6005) (width 0.5) (layer B.Cu) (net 1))
 (segment (start 142.748 38.735) (end 142.748 41.275) (width 0.5) (layer B.Cu) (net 3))
 (segment (start 142.748 41.275) (end 142.748 42.6005) (width 0.5) (layer B.Cu) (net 3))
 (segment (start 145.3166 55.9498) (end 145.3166 55.839798) (width 0.3) (layer B.Cu) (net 3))
 (segment (start 145.3166 55.839798) (end 144.366599 54.889797) (width 0.3) (layer B.Cu) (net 3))
 (segment (start 144.366599 54.889797) (end 144.366599 52.899799) (width 0.3) (layer B.Cu) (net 3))
 (segment (start 144.366599 46.759099) (end 144.366599 52.899799) (width 0.5) (layer B.Cu) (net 3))
 (segment (start 140.208 42.6005) (end 144.366599 46.759099) (width 0.5) (layer B.Cu) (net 3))
 (segment (start 142.748 42.6005) (end 145.3166 45.1691) (width 0.5) (layer B.Cu) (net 3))
 (segment (start 145.3166 45.1691) (end 145.3166 52.7998) (width 0.5) (layer B.Cu) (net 3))
 (segment (start 147.828 38.735) (end 147.828 41.275) (width 0.5) (layer B.Cu) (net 5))
 (segment (start 147.3136 55.9498) (end 146.366599 55.002799) (width 0.3) (layer B.Cu) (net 5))
 (segment (start 146.366599 55.002799) (end 146.366599 52.899799) (width 0.3) (layer B.Cu) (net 5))
 (segment (start 147.3166 55.9498) (end 147.3136 55.9498) (width 0.3) (layer B.Cu) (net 5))
 (segment (start 146.366599 43.679099) (end 146.366599 52.899799) (width 0.5) (layer B.Cu) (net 5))
 (segment (start 145.288 42.6005) (end 146.366599 43.679099) (width 0.5) (layer B.Cu) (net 5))
 (segment (start 147.3166 53.9498) (end 147.3166 53.7938) (width 0.4) (layer B.Cu) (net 6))
 (segment (start 147.828 53.4384) (end 147.3166 53.9498) (width 0.5) (layer B.Cu) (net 6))
 (segment (start 147.828 41.275) (end 147.828 53.4384) (width 0.5) (layer B.Cu) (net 6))
 (segment (start 145.288 38.735) (end 145.288 41.275) (width 0.5) (layer B.Cu) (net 6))
 (segment (start 145.288 41.275) (end 145.288 42.6005) (width 0.5) (layer B.Cu) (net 6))
 (segment (start 145.3166 52.7998) (end 145.3166 53.9498) (width 0.5) (layer B.Cu) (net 4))
 (segment (start 140.208 38.735) (end 140.208 41.275) (width 0.5) (layer B.Cu) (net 4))
 (segment (start 140.208 41.275) (end 140.208 42.6005) (width 0.5) (layer B.Cu) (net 4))
 (segment (start 118.0846 38.7858) (end 118.0846 41.3258) (width 0.5) (layer B.Cu) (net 9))
 (segment (start 118.0846 52.6818) (end 116.8166 53.9498) (width 0.5) (layer B.Cu) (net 9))
 (segment (start 118.0846 41.3258) (end 118.0846 52.6818) (width 0.5) (layer B.Cu) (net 9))
 (segment (start 120.6246 38.7858) (end 120.6246 41.3258) (width 0.5) (layer B.Cu) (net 10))
 (segment (start 120.6246 53.2918) (end 119.9666 53.9498) (width 0.5) (layer B.Cu) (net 10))
 (segment (start 120.6246 41.3258) (end 120.6246 53.2918) (width 0.5) (layer B.Cu) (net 10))
 (segment (start 116.8166 57.0998) (end 116.8166 55.9498) (width 0.5) (layer B.Cu) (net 10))
 (segment (start 117.2224 57.5056) (end 116.8166 57.0998) (width 0.5) (layer B.Cu) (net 10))
 (segment (start 119.9388 57.5056) (end 117.2224 57.5056) (width 0.5) (layer B.Cu) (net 10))
 (segment (start 121.385497 56.058903) (end 119.9388 57.5056) (width 0.5) (layer B.Cu) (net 10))
 (segment (start 122.809 45.5469) (end 122.809 54.6354) (width 0.5) (layer B.Cu) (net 10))
 (segment (start 122.809 54.6354) (end 121.385497 56.058903) (width 0.5) (layer B.Cu) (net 10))
 (segment (start 125.7046 42.6513) (end 122.809 45.5469) (width 0.5) (layer B.Cu) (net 10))
 (segment (start 125.7046 41.3258) (end 125.7046 42.6513) (width 0.5) (layer B.Cu) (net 11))
 (segment (start 119.9666 53.9498) (end 118.8166 53.9498) (width 0.5) (layer B.Cu) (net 11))
 (segment (start 125.7046 38.7858) (end 125.7046 41.3258) (width 0.5) (layer B.Cu) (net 11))
 (segment (start 121.561267 54.355133) (end 119.9666 55.9498) (width 0.5) (layer B.Cu) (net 12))
 (segment (start 123.1646 41.3258) (end 123.1646 42.6513) (width 0.5) (layer B.Cu) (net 12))
 (segment (start 121.561267 44.254633) (end 121.561267 54.355133) (width 0.5) (layer B.Cu) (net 12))
 (segment (start 123.1646 42.6513) (end 121.561267 44.254633) (width 0.5) (layer B.Cu) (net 12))
 (segment (start 123.1646 38.7858) (end 123.1646 41.3258) (width 0.5) (layer B.Cu) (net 12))
 (segment (start 119.9666 55.9498) (end 118.8166 55.9498) (width 0.5) (layer B.Cu) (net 12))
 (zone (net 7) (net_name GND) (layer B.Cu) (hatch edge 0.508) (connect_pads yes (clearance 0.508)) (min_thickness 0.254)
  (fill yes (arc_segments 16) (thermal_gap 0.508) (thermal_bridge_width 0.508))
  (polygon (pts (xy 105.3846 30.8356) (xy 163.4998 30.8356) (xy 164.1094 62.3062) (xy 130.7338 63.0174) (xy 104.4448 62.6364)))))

